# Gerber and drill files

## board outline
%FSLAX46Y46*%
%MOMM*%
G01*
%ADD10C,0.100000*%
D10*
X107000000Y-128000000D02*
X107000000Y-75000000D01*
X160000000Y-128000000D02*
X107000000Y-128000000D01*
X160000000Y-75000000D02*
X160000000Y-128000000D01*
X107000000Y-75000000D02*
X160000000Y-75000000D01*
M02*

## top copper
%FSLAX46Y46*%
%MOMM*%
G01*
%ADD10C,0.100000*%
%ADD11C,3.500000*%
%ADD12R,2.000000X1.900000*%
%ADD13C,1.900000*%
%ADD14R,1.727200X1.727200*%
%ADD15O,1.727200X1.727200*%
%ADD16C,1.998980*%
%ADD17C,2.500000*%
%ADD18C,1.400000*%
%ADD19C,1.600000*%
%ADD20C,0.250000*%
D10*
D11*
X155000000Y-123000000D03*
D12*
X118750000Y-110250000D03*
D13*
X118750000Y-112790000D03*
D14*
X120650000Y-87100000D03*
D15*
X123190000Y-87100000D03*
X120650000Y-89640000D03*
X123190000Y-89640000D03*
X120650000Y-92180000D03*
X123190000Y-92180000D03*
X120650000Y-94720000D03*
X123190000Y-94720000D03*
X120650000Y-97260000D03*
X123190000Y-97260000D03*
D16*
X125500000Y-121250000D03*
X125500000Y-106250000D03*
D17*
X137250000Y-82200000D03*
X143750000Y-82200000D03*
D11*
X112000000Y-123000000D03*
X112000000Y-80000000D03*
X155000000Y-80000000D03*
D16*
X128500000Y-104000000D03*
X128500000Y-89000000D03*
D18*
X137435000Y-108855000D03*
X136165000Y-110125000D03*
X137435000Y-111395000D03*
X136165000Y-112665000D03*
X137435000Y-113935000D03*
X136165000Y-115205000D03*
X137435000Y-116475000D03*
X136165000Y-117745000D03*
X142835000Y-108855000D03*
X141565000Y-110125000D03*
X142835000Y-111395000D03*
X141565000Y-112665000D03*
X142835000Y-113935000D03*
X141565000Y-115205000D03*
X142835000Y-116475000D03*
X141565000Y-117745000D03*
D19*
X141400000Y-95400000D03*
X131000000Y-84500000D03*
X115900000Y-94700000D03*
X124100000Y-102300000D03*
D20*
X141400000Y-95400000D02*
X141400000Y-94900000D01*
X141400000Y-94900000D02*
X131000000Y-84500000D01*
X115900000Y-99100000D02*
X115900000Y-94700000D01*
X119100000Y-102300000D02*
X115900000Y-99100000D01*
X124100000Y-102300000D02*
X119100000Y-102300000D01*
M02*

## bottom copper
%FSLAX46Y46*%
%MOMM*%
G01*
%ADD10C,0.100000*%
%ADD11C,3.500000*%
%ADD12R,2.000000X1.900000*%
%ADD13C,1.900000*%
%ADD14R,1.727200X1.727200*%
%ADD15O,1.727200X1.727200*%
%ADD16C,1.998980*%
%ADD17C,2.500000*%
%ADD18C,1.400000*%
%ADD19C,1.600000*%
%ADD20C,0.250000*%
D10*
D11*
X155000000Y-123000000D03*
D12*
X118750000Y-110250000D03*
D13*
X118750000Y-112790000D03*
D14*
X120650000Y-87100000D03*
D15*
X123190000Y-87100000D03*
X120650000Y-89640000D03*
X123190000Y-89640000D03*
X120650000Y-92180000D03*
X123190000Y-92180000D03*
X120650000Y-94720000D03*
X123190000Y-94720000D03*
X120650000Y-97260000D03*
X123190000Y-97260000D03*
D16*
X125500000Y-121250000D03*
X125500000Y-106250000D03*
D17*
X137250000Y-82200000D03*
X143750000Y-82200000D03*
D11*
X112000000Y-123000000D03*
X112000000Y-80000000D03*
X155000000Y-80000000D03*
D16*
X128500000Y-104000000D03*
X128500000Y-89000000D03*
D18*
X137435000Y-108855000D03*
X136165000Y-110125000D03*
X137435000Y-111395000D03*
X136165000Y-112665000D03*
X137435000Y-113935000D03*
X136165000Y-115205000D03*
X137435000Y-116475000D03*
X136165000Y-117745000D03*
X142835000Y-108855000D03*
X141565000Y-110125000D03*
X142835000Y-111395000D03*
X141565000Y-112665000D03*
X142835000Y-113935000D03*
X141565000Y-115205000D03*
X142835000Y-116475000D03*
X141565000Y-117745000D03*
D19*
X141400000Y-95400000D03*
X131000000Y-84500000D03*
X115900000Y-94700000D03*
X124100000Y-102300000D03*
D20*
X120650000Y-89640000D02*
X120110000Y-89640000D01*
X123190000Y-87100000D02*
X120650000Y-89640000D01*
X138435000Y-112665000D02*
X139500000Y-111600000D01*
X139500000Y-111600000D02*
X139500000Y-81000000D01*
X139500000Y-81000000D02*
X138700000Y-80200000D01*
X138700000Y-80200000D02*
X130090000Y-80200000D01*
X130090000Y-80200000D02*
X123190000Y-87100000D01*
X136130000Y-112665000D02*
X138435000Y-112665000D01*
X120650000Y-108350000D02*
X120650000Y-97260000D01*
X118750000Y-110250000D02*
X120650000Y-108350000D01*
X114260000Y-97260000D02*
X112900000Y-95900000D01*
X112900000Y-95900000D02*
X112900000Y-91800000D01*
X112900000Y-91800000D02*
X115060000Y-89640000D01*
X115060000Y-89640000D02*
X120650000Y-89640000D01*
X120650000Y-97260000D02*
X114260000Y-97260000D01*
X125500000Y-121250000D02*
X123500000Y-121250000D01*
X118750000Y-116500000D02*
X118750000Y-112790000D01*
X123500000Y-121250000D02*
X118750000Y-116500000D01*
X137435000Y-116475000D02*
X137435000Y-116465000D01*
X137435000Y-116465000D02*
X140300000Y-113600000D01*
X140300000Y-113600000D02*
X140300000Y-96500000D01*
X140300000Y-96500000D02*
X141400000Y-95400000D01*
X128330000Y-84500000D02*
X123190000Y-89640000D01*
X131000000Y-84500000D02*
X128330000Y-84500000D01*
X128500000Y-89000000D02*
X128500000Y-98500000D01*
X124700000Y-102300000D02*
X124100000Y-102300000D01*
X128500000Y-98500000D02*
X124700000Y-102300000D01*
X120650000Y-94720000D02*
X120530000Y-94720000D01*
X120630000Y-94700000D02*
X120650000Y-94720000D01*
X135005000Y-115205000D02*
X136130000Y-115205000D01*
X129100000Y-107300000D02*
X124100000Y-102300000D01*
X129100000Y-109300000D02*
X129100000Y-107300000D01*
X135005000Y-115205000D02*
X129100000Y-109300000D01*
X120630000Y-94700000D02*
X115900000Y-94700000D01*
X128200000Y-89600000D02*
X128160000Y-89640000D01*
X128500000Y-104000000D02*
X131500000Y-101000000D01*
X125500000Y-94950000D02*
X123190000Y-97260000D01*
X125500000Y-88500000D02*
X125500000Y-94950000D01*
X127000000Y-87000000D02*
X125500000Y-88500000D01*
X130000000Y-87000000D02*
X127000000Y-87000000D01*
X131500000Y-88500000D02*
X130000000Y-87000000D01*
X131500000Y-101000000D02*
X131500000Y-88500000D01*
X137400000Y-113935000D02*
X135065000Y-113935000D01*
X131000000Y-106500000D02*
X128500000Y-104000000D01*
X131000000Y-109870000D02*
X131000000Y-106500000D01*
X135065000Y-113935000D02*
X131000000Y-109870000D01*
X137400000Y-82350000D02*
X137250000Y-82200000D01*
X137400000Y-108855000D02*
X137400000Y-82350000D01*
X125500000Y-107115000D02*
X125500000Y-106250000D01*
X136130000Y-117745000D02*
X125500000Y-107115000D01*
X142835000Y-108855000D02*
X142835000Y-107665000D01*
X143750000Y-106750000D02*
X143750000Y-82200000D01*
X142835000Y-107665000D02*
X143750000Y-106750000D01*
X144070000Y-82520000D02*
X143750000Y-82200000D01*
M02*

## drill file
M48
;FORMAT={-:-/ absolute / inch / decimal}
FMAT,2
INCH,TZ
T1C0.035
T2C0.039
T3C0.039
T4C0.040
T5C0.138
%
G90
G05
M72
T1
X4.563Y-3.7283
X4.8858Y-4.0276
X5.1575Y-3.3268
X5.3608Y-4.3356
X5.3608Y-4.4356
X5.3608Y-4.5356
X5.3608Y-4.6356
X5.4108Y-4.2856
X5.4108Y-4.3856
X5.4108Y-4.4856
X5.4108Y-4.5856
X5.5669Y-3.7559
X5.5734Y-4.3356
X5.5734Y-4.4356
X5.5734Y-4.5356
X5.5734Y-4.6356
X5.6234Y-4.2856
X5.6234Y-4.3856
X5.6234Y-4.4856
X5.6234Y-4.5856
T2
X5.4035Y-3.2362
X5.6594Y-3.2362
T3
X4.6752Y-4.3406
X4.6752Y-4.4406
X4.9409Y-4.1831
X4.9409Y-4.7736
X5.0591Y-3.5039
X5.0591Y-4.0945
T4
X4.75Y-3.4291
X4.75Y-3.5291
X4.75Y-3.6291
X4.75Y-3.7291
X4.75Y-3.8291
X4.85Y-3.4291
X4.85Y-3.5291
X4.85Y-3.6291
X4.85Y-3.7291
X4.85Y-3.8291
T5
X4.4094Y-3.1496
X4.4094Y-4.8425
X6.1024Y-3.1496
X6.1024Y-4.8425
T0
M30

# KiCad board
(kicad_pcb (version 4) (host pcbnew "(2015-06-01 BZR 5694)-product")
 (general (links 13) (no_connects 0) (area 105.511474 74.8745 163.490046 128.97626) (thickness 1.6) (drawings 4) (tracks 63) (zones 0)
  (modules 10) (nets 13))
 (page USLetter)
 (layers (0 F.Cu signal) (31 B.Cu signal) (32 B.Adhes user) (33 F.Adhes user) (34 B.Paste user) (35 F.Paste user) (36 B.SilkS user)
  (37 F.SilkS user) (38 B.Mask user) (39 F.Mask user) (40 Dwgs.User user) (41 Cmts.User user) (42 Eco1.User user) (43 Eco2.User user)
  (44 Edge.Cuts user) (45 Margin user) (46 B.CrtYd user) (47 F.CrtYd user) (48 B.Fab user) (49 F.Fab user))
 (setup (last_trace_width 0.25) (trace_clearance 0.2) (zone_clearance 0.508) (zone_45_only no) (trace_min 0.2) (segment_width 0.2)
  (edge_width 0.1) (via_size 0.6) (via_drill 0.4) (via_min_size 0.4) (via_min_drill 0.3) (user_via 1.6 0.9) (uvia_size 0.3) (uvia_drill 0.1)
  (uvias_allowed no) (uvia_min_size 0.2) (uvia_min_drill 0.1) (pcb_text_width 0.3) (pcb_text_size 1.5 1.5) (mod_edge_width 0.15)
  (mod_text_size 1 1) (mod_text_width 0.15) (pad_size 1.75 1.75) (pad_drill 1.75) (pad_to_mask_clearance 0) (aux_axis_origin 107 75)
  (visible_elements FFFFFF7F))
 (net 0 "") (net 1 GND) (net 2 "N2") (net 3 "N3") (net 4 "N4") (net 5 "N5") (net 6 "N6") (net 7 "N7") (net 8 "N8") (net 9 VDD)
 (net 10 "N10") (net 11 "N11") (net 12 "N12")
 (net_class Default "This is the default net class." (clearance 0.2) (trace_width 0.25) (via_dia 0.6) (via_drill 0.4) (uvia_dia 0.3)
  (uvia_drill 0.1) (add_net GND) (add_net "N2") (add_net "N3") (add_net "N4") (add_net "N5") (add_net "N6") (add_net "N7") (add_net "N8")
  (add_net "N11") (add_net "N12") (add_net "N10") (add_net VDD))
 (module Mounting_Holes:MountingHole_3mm (layer F.Cu) (at 155 123)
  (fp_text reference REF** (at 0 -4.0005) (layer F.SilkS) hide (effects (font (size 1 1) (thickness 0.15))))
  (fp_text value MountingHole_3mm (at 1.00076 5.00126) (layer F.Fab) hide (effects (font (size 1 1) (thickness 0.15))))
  (pad "" thru_hole circle (at 0 0) (size 3.5 3.5) (drill 3.5) (layers *.Cu *.Mask F.SilkS)))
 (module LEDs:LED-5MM (layer F.Cu) (at 118.75 110.25 270)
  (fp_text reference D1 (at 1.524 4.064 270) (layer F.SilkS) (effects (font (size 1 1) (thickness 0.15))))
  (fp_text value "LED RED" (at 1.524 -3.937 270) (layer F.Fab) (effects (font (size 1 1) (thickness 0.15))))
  (pad 1 thru_hole rect (at 0 0) (size 2 1.9) (drill 1.00076) (layers *.Cu *.Mask F.SilkS) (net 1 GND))
  (pad 2 thru_hole circle (at 2.54 0 270) (size 1.9 1.9) (drill 1.00076) (layers *.Cu *.Mask F.SilkS) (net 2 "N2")))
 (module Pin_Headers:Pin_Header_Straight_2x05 (layer F.Cu) (at 120.65 87.1)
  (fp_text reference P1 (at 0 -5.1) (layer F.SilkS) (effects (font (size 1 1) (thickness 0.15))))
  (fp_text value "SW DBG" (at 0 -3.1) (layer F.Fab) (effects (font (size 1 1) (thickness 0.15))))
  (pad 1 thru_hole rect (at 0 0) (size 1.7272 1.7272) (drill 1.016) (layers *.Cu *.Mask F.SilkS) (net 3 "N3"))
  (pad 2 thru_hole oval (at 2.54 0) (size 1.7272 1.7272) (drill 1.016) (layers *.Cu *.Mask F.SilkS) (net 1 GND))
  (pad 3 thru_hole oval (at 0 2.54) (size 1.7272 1.7272) (drill 1.016) (layers *.Cu *.Mask F.SilkS) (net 1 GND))
  (pad 4 thru_hole oval (at 2.54 2.54) (size 1.7272 1.7272) (drill 1.016) (layers *.Cu *.Mask F.SilkS) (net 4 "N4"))
  (pad 5 thru_hole oval (at 0 5.08) (size 1.7272 1.7272) (drill 1.016) (layers *.Cu *.Mask F.SilkS) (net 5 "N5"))
  (pad 6 thru_hole oval (at 2.54 5.08) (size 1.7272 1.7272) (drill 1.016) (layers *.Cu *.Mask F.SilkS) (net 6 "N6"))
  (pad 7 thru_hole oval (at 0 7.62) (size 1.7272 1.7272) (drill 1.016) (layers *.Cu *.Mask F.SilkS) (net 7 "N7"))
  (pad 8 thru_hole oval (at 2.54 7.62) (size 1.7272 1.7272) (drill 1.016) (layers *.Cu *.Mask F.SilkS) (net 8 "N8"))
  (pad 9 thru_hole oval (at 0 10.16) (size 1.7272 1.7272) (drill 1.016) (layers *.Cu *.Mask F.SilkS) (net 1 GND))
  (pad 10 thru_hole oval (at 2.54 10.16) (size 1.7272 1.7272) (drill 1.016) (layers *.Cu *.Mask F.SilkS) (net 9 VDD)))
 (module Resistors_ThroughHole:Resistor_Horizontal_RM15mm (layer F.Cu) (at 125.5 113.75 90)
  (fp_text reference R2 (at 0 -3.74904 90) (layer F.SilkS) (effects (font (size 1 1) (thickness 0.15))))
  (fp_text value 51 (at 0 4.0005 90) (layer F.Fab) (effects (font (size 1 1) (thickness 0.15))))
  (pad 1 thru_hole circle (at -7.5 0 90) (size 1.99898 1.99898) (drill 1.00076) (layers *.Cu *.SilkS *.Mask) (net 2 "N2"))
  (pad 2 thru_hole circle (at 7.5 0 90) (size 1.99898 1.99898) (drill 1.00076) (layers *.Cu *.SilkS *.Mask) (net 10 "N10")))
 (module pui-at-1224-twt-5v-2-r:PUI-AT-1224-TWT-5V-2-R (layer F.Cu) (at 140.5 82.2)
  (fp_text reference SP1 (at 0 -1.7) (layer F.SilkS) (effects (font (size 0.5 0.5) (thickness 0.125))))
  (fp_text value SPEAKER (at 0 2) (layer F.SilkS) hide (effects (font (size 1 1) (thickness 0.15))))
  (pad 1 thru_hole circle (at -3.25 0) (size 2.5 2.5) (drill 1) (layers *.Cu *.Mask F.SilkS) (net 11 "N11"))
  (pad 2 thru_hole circle (at 3.25 0) (size 2.5 2.5) (drill 1) (layers *.Cu *.Mask F.SilkS) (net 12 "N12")))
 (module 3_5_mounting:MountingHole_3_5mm (layer F.Cu) (at 112 123)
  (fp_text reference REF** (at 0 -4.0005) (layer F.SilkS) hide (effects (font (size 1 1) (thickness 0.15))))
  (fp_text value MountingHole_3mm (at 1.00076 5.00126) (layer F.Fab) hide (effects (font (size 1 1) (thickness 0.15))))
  (pad "" thru_hole circle (at 0 0) (size 3.5 3.5) (drill 3.5) (layers *.Cu *.Mask F.SilkS)))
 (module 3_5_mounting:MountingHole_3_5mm (layer F.Cu) (at 112 80)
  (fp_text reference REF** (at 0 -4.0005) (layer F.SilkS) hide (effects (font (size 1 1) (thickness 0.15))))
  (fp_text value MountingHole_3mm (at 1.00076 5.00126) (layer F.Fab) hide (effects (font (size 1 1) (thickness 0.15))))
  (pad "" thru_hole circle (at 0 0) (size 3.5 3.5) (drill 3.5) (layers *.Cu *.Mask F.SilkS)))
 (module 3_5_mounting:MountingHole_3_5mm (layer F.Cu) (at 155 80)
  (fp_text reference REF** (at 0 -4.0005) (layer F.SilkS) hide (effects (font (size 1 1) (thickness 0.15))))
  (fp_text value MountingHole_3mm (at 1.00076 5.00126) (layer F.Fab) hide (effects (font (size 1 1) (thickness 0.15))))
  (pad "" thru_hole circle (at 0 0) (size 3.5 3.5) (drill 3.5) (layers *.Cu *.Mask F.SilkS)))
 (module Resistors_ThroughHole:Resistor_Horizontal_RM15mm (layer F.Cu) (at 128.5 96.5 90)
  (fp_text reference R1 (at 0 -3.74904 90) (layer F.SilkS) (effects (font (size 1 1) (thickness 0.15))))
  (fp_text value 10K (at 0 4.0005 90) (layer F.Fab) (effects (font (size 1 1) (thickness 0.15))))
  (pad 1 thru_hole circle (at -7.5 0 90) (size 1.99898 1.99898) (drill 1.00076) (layers *.Cu *.SilkS *.Mask) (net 9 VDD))
  (pad 2 thru_hole circle (at 7.5 0 90) (size 1.99898 1.99898) (drill 1.00076) (layers *.Cu *.SilkS *.Mask) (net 7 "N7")))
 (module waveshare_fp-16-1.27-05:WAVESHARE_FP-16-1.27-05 (layer F.Cu) (at 139.5 113.3)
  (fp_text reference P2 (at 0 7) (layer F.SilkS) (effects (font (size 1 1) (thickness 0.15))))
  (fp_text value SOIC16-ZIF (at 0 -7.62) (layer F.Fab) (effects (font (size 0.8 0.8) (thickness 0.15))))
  (pad 1 thru_hole circle (at -2.065 -4.445) (size 1.4 1.4) (drill 0.9) (layers *.Cu *.Mask F.SilkS) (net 11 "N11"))
  (pad 2 thru_hole circle (at -3.335 -3.175) (size 1.4 1.4) (drill 0.9) (layers *.Cu *.Mask F.SilkS))
  (pad 3 thru_hole circle (at -2.065 -1.905) (size 1.4 1.4) (drill 0.9) (layers *.Cu *.Mask F.SilkS))
  (pad 4 thru_hole circle (at -3.335 -0.635) (size 1.4 1.4) (drill 0.9) (layers *.Cu *.Mask F.SilkS) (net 1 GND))
  (pad 5 thru_hole circle (at -2.065 0.635) (size 1.4 1.4) (drill 0.9) (layers *.Cu *.Mask F.SilkS) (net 9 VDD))
  (pad 6 thru_hole circle (at -3.335 1.905) (size 1.4 1.4) (drill 0.9) (layers *.Cu *.Mask F.SilkS) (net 7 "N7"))
  (pad 7 thru_hole circle (at -2.065 3.175) (size 1.4 1.4) (drill 0.9) (layers *.Cu *.Mask F.SilkS) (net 4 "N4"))
  (pad 8 thru_hole circle (at -3.335 4.445) (size 1.4 1.4) (drill 0.9) (layers *.Cu *.Mask F.SilkS) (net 10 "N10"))
  (pad 16 thru_hole circle (at 3.335 -4.445) (size 1.4 1.4) (drill 0.9) (layers *.Cu *.Mask F.SilkS) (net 12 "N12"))
  (pad 15 thru_hole circle (at 2.065 -3.175) (size 1.4 1.4) (drill 0.9) (layers *.Cu *.Mask F.SilkS))
  (pad 14 thru_hole circle (at 3.335 -1.905) (size 1.4 1.4) (drill 0.9) (layers *.Cu *.Mask F.SilkS))
  (pad 13 thru_hole circle (at 2.065 -0.635) (size 1.4 1.4) (drill 0.9) (layers *.Cu *.Mask F.SilkS))
  (pad 12 thru_hole circle (at 3.335 0.635) (size 1.4 1.4) (drill 0.9) (layers *.Cu *.Mask F.SilkS))
  (pad 11 thru_hole circle (at 2.065 1.905) (size 1.4 1.4) (drill 0.9) (layers *.Cu *.Mask F.SilkS))
  (pad 10 thru_hole circle (at 3.335 3.175) (size 1.4 1.4) (drill 0.9) (layers *.Cu *.Mask F.SilkS))
  (pad 9 thru_hole circle (at 2.065 4.445) (size 1.4 1.4) (drill 0.9) (layers *.Cu *.Mask F.SilkS)))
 (gr_line (start 107 128) (end 107 75) (angle 90) (layer Edge.Cuts) (width 0.1))
 (gr_line (start 160 128) (end 107 128) (angle 90) (layer Edge.Cuts) (width 0.1))
 (gr_line (start 160 75) (end 160 128) (angle 90) (layer Edge.Cuts) (width 0.1))
 (gr_line (start 107 75) (end 160 75) (angle 90) (layer Edge.Cuts) (width 0.1))
 (segment (start 120.65 89.64) (end 120.11 89.64) (width 0.25) (layer B.Cu) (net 1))
 (segment (start 123.19 87.1) (end 120.65 89.64) (width 0.25) (layer B.Cu) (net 1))
 (segment (start 138.435 112.665) (end 139.5 111.6) (width 0.25) (layer B.Cu) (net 1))
 (segment (start 139.5 111.6) (end 139.5 81) (width 0.25) (layer B.Cu) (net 1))
 (segment (start 139.5 81) (end 138.7 80.2) (width 0.25) (layer B.Cu) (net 1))
 (segment (start 138.7 80.2) (end 130.09 80.2) (width 0.25) (layer B.Cu) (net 1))
 (segment (start 130.09 80.2) (end 123.19 87.1) (width 0.25) (layer B.Cu) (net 1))
 (segment (start 136.13 112.665) (end 138.435 112.665) (width 0.25) (layer B.Cu) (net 1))
 (segment (start 120.65 108.35) (end 120.65 97.26) (width 0.25) (layer B.Cu) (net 1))
 (segment (start 118.75 110.25) (end 120.65 108.35) (width 0.25) (layer B.Cu) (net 1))
 (segment (start 114.26 97.26) (end 112.9 95.9) (width 0.25) (layer B.Cu) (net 1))
 (segment (start 112.9 95.9) (end 112.9 91.8) (width 0.25) (layer B.Cu) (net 1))
 (segment (start 112.9 91.8) (end 115.06 89.64) (width 0.25) (layer B.Cu) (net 1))
 (segment (start 115.06 89.64) (end 120.65 89.64) (width 0.25) (layer B.Cu) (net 1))
 (segment (start 120.65 97.26) (end 114.26 97.26) (width 0.25) (layer B.Cu) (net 1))
 (segment (start 125.5 121.25) (end 123.5 121.25) (width 0.25) (layer B.Cu) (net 2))
 (segment (start 118.75 116.5) (end 118.75 112.79) (width 0.25) (layer B.Cu) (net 2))
 (segment (start 123.5 121.25) (end 118.75 116.5) (width 0.25) (layer B.Cu) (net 2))
 (segment (start 137.435 116.475) (end 137.435 116.465) (width 0.25) (layer B.Cu) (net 4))
 (segment (start 137.435 116.465) (end 140.3 113.6) (width 0.25) (layer B.Cu) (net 4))
 (segment (start 140.3 113.6) (end 140.3 96.5) (width 0.25) (layer B.Cu) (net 4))
 (segment (start 140.3 96.5) (end 141.4 95.4) (width 0.25) (layer B.Cu) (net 4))
 (segment (start 141.4 95.4) (end 141.4 94.9) (width 0.25) (layer F.Cu) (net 4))
 (via (at 141.4 95.4) (size 1.6) (drill 0.9) (layers F.Cu B.Cu) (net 4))
 (segment (start 128.33 84.5) (end 123.19 89.64) (width 0.25) (layer B.Cu) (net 4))
 (segment (start 131 84.5) (end 128.33 84.5) (width 0.25) (layer B.Cu) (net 4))
 (via (at 131 84.5) (size 1.6) (drill 0.9) (layers F.Cu B.Cu) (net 4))
 (segment (start 141.4 94.9) (end 131 84.5) (width 0.25) (layer F.Cu) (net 4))
 (segment (start 128.5 89) (end 128.5 98.5) (width 0.25) (layer B.Cu) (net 7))
 (segment (start 124.7 102.3) (end 124.1 102.3) (width 0.25) (layer B.Cu) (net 7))
 (segment (start 128.5 98.5) (end 124.7 102.3) (width 0.25) (layer B.Cu) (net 7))
 (segment (start 120.65 94.72) (end 120.53 94.72) (width 0.25) (layer B.Cu) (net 7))
 (segment (start 120.63 94.7) (end 120.65 94.72) (width 0.25) (layer B.Cu) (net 7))
 (segment (start 135.005 115.205) (end 136.13 115.205) (width 0.25) (layer B.Cu) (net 7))
 (via (at 115.9 94.7) (size 1.6) (drill 0.9) (layers F.Cu B.Cu) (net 7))
 (segment (start 115.9 99.1) (end 115.9 94.7) (width 0.25) (layer F.Cu) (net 7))
 (segment (start 119.1 102.3) (end 115.9 99.1) (width 0.25) (layer F.Cu) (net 7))
 (segment (start 124.1 102.3) (end 119.1 102.3) (width 0.25) (layer F.Cu) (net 7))
 (via (at 124.1 102.3) (size 1.6) (drill 0.9) (layers F.Cu B.Cu) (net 7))
 (segment (start 129.1 107.3) (end 124.1 102.3) (width 0.25) (layer B.Cu) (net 7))
 (segment (start 129.1 109.3) (end 129.1 107.3) (width 0.25) (layer B.Cu) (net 7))
 (segment (start 135.005 115.205) (end 129.1 109.3) (width 0.25) (layer B.Cu) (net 7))
 (segment (start 120.63 94.7) (end 115.9 94.7) (width 0.25) (layer B.Cu) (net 7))
 (segment (start 128.2 89.6) (end 128.16 89.64) (width 0.25) (layer B.Cu) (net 7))
 (segment (start 128.5 104) (end 131.5 101) (width 0.25) (layer B.Cu) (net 9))
 (segment (start 125.5 94.95) (end 123.19 97.26) (width 0.25) (layer B.Cu) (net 9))
 (segment (start 125.5 88.5) (end 125.5 94.95) (width 0.25) (layer B.Cu) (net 9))
 (segment (start 127 87) (end 125.5 88.5) (width 0.25) (layer B.Cu) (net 9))
 (segment (start 130 87) (end 127 87) (width 0.25) (layer B.Cu) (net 9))
 (segment (start 131.5 88.5) (end 130 87) (width 0.25) (layer B.Cu) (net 9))
 (segment (start 131.5 101) (end 131.5 88.5) (width 0.25) (layer B.Cu) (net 9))
 (segment (start 137.4 113.935) (end 135.065 113.935) (width 0.25) (layer B.Cu) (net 9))
 (segment (start 131 106.5) (end 128.5 104) (width 0.25) (layer B.Cu) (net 9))
 (segment (start 131 109.87) (end 131 106.5) (width 0.25) (layer B.Cu) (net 9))
 (segment (start 135.065 113.935) (end 131 109.87) (width 0.25) (layer B.Cu) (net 9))
 (segment (start 137.4 82.35) (end 137.25 82.2) (width 0.25) (layer B.Cu) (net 11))
 (segment (start 137.4 108.855) (end 137.4 82.35) (width 0.25) (layer B.Cu) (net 11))
 (segment (start 125.5 107.115) (end 125.5 106.25) (width 0.25) (layer B.Cu) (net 10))
 (segment (start 136.13 117.745) (end 125.5 107.115) (width 0.25) (layer B.Cu) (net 10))
 (segment (start 142.835 108.855) (end 142.835 107.665) (width 0.25) (layer B.Cu) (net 12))
 (segment (start 143.75 106.75) (end 143.75 82.2) (width 0.25) (layer B.Cu) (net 12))
 (segment (start 142.835 107.665) (end 143.75 106.75) (width 0.25) (layer B.Cu) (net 12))
 (segment (start 144.07 82.52) (end 143.75 82.2) (width 0.25) (layer B.Cu) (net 12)))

